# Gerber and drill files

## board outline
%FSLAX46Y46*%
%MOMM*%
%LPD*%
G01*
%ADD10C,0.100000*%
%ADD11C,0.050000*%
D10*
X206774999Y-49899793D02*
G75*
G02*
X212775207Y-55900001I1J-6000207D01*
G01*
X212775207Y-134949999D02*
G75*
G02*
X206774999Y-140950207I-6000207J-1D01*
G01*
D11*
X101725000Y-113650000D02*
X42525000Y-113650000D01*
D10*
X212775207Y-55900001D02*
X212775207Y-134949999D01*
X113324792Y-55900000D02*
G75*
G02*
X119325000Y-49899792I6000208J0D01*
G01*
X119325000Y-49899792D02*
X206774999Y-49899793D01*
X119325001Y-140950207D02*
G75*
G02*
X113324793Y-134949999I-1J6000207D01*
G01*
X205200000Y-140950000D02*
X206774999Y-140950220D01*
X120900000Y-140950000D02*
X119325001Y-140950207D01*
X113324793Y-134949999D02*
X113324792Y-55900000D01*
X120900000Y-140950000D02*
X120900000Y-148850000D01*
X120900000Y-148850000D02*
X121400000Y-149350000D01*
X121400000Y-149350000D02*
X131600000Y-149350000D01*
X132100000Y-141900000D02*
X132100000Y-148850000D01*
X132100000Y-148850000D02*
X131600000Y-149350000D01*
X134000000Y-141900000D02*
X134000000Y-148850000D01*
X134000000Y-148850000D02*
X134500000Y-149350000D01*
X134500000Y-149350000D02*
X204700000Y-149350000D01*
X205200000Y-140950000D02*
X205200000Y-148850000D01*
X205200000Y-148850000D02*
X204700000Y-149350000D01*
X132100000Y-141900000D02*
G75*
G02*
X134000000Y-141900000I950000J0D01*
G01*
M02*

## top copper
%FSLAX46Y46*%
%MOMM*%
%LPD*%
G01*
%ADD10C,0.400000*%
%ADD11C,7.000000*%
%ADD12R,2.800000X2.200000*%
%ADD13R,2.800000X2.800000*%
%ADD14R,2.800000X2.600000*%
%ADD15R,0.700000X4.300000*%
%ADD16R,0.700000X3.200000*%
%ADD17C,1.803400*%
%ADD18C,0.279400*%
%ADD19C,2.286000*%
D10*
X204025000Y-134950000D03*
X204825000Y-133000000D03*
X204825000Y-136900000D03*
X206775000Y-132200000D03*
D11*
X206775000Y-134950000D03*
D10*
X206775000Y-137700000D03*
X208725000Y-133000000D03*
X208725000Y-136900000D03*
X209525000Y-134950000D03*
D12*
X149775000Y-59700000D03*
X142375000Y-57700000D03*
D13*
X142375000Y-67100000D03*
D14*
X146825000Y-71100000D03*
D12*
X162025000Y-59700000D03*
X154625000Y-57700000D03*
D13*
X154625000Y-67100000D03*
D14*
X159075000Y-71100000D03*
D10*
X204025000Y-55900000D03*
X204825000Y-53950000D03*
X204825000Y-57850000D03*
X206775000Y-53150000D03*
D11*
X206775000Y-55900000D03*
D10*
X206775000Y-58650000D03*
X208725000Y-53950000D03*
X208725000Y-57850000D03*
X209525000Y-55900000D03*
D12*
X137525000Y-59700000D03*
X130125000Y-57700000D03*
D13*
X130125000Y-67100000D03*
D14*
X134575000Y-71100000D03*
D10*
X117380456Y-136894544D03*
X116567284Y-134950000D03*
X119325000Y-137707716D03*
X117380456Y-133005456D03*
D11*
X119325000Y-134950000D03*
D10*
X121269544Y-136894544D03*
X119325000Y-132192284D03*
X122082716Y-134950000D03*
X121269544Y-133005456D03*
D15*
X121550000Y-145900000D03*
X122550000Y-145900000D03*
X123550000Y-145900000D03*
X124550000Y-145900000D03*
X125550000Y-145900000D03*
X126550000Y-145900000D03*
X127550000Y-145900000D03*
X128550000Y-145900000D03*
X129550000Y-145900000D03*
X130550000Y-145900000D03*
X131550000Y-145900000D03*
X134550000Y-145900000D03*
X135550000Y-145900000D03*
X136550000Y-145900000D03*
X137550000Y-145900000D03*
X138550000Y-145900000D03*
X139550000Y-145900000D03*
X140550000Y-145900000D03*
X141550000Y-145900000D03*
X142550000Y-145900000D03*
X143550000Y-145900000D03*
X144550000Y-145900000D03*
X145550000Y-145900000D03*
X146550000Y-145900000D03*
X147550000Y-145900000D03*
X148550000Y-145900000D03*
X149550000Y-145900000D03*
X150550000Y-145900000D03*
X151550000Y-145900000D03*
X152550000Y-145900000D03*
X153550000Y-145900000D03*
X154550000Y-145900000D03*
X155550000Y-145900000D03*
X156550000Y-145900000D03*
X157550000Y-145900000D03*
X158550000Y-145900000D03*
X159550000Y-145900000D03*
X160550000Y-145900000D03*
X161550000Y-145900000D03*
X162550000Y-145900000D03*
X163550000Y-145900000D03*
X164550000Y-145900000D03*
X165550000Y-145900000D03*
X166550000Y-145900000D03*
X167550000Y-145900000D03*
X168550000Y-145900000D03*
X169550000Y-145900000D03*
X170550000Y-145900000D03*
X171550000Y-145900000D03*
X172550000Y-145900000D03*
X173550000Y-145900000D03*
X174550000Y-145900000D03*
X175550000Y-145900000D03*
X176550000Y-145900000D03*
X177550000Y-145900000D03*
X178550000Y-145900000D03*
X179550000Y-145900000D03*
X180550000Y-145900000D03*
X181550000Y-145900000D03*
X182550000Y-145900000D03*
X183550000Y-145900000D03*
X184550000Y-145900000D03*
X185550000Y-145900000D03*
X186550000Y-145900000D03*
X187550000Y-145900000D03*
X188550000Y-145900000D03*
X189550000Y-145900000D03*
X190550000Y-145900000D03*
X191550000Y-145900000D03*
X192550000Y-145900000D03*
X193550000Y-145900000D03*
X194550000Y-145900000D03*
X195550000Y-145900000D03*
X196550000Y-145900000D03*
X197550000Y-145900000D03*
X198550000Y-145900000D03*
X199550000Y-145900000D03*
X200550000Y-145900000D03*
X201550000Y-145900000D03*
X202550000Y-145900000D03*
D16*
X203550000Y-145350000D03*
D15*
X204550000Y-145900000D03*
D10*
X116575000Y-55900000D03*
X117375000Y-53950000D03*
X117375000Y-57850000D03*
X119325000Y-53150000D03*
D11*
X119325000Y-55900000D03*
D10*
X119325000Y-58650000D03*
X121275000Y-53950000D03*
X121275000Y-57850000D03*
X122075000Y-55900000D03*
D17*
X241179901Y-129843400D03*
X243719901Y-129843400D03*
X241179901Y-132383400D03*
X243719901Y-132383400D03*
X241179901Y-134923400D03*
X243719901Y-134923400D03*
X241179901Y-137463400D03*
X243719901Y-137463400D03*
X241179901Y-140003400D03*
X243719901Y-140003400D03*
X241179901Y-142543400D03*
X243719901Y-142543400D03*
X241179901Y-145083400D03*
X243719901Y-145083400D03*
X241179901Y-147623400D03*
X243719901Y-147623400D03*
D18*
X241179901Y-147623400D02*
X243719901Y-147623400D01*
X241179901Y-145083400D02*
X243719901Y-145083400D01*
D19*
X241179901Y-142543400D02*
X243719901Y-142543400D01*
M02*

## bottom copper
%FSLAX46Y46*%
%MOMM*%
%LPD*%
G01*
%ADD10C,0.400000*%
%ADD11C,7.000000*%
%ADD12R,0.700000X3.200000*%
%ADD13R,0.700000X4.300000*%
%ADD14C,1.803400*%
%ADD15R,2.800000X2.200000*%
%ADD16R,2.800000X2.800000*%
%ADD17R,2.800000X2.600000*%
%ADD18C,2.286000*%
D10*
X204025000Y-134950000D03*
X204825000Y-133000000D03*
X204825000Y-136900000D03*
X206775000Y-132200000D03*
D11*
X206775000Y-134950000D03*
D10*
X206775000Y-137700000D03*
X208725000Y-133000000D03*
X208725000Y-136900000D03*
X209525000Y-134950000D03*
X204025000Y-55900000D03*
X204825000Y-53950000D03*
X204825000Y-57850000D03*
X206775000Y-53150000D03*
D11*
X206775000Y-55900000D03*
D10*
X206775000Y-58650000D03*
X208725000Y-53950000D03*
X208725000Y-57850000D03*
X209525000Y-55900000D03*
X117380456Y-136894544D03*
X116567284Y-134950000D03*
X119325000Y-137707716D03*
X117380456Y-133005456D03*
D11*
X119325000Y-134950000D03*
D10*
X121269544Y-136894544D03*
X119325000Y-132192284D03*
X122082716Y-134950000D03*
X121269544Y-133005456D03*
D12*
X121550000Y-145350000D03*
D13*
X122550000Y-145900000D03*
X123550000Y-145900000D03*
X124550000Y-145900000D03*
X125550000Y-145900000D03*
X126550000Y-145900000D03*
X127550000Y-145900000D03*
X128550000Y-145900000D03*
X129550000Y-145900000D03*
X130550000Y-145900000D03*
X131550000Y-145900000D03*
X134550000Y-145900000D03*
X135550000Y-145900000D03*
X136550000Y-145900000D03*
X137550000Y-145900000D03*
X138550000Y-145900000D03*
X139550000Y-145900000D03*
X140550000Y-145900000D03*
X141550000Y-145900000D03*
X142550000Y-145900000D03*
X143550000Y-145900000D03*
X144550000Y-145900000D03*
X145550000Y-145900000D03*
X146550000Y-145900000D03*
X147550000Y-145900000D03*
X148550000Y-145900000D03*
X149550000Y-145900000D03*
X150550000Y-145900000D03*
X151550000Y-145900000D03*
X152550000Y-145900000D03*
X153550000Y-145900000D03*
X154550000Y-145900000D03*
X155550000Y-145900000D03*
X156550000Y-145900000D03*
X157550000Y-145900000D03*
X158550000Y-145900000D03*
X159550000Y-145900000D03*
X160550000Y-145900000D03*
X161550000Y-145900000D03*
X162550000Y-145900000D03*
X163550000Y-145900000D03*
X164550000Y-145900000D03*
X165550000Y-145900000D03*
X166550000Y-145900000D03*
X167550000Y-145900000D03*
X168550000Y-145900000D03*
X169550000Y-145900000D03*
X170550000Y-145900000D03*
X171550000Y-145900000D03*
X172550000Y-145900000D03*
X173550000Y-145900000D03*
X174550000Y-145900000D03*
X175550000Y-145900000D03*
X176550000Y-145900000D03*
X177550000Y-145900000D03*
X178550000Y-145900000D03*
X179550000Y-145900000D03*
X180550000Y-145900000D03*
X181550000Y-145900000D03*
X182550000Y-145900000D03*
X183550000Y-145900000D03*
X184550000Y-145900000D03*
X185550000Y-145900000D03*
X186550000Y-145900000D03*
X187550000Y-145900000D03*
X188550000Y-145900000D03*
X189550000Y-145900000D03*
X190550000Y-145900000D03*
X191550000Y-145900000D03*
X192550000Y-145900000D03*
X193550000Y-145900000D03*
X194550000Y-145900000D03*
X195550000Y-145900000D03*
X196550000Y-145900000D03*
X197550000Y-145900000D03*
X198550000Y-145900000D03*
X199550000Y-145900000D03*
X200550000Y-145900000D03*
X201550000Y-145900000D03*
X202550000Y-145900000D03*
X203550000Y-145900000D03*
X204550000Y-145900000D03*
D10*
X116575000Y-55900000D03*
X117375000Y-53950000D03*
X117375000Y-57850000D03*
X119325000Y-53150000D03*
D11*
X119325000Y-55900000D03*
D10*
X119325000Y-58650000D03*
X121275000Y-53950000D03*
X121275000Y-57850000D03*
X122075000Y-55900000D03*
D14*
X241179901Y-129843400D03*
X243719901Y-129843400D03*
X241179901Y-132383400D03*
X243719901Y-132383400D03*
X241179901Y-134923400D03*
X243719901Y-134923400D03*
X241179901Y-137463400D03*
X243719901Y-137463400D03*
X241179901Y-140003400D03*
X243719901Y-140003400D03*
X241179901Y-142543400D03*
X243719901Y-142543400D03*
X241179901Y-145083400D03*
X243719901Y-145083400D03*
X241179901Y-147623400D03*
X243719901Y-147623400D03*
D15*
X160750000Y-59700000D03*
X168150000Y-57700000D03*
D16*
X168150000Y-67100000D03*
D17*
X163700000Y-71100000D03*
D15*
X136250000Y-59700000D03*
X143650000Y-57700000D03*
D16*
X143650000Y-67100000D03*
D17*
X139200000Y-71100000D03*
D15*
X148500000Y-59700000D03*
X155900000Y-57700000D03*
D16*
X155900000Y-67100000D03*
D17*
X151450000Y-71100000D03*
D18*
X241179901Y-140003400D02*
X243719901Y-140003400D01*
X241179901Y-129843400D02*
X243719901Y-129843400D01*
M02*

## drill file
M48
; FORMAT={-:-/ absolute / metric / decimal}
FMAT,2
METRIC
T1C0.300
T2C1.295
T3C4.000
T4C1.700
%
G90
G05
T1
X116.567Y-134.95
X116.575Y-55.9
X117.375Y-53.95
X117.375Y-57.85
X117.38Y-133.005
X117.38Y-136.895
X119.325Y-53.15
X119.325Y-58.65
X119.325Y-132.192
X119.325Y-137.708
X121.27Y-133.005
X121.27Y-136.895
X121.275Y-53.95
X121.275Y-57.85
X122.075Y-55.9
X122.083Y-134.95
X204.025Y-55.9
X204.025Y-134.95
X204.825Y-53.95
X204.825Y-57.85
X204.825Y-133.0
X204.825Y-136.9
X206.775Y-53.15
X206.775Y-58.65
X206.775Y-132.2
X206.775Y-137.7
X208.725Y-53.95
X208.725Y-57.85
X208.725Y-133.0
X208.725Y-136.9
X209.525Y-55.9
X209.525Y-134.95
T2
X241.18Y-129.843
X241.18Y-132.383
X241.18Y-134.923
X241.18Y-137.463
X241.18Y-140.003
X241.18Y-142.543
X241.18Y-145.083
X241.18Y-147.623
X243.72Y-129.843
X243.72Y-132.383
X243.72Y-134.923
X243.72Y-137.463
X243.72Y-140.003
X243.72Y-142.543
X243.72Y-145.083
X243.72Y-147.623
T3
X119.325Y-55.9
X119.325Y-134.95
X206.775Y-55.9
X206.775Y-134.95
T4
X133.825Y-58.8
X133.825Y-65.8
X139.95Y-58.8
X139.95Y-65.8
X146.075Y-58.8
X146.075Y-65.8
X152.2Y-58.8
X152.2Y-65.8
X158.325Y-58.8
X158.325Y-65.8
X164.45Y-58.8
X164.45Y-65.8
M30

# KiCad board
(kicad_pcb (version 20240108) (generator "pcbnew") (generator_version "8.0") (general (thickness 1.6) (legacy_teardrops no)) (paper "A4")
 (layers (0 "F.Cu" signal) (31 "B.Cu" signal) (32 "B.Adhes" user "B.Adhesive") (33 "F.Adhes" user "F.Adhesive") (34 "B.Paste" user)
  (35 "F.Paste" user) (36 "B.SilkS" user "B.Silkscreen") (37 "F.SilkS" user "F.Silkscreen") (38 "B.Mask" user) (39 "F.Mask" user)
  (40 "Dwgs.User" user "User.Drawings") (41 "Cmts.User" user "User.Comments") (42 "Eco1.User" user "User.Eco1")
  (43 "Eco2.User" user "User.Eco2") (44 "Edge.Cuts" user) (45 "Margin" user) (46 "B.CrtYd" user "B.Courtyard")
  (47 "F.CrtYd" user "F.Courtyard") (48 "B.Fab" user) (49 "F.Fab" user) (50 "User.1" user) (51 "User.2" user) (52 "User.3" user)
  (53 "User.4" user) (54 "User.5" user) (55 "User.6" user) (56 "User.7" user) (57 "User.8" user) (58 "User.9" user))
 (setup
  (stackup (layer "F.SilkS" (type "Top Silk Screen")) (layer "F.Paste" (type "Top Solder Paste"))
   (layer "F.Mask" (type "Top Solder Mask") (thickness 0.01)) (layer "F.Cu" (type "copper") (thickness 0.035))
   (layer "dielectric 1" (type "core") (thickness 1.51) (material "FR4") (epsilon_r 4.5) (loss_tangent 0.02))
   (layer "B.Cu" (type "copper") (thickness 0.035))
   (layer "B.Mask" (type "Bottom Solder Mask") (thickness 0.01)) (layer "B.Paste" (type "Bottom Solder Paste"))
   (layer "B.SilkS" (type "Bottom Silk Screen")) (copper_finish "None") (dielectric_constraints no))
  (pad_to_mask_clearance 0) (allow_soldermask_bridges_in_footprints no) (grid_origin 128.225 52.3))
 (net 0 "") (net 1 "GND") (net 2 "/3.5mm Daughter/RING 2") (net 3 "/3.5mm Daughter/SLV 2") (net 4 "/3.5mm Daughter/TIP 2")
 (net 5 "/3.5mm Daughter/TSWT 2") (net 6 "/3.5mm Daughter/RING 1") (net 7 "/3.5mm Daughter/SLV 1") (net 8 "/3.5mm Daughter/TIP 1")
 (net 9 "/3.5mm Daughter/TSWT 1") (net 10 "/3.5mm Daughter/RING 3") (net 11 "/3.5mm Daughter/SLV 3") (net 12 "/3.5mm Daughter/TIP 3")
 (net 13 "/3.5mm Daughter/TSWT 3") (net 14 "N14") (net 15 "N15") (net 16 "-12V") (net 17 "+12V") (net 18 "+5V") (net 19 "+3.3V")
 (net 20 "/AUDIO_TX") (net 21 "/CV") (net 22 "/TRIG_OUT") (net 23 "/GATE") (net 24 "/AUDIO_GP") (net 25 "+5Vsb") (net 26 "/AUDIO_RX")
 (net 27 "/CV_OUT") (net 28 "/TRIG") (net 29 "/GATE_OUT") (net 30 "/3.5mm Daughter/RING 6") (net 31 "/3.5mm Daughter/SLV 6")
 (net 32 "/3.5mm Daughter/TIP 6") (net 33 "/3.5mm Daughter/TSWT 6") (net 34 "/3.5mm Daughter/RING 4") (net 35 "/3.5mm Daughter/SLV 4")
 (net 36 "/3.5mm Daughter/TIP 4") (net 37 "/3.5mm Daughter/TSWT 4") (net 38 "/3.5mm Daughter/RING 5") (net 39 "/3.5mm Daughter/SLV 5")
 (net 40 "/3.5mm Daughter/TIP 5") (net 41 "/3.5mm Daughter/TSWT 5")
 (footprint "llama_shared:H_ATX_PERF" (layer "F.Cu") (at 206.775 134.95)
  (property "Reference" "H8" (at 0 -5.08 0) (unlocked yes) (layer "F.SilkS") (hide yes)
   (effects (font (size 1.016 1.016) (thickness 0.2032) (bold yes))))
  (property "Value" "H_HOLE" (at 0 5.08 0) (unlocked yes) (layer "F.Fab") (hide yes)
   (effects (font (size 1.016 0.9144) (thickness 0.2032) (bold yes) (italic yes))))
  (pad "1" thru_hole circle (at -2.75 0) (size 0.4 0.4) (drill 0.3) (layers "*.Cu" "*.Mask") (remove_unused_layers no) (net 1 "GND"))
  (pad "1" thru_hole circle (at -1.95 -1.95) (size 0.4 0.4) (drill 0.3) (layers "*.Cu" "*.Mask") (remove_unused_layers no) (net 1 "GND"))
  (pad "1" thru_hole circle (at -1.95 1.95) (size 0.4 0.4) (drill 0.3) (layers "*.Cu" "*.Mask") (remove_unused_layers no) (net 1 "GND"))
  (pad "1" thru_hole circle (at 0 -2.75) (size 0.4 0.4) (drill 0.3) (layers "*.Cu" "*.Mask") (remove_unused_layers no) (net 1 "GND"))
  (pad "1" thru_hole circle (at 0 0) (size 7 7) (drill 4) (layers "*.Cu" "*.Mask") (remove_unused_layers no) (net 1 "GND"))
  (pad "1" thru_hole circle (at 0 2.75) (size 0.4 0.4) (drill 0.3) (layers "*.Cu" "*.Mask") (remove_unused_layers no) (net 1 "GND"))
  (pad "1" thru_hole circle (at 1.95 -1.95) (size 0.4 0.4) (drill 0.3) (layers "*.Cu" "*.Mask") (remove_unused_layers no) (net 1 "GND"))
  (pad "1" thru_hole circle (at 1.95 1.95) (size 0.4 0.4) (drill 0.3) (layers "*.Cu" "*.Mask") (remove_unused_layers no) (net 1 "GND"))
  (pad "1" thru_hole circle (at 2.75 0) (size 0.4 0.4) (drill 0.3) (layers "*.Cu" "*.Mask") (remove_unused_layers no) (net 1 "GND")))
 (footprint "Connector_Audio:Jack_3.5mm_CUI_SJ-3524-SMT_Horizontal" (layer "F.Cu") (at 146.075 61.3)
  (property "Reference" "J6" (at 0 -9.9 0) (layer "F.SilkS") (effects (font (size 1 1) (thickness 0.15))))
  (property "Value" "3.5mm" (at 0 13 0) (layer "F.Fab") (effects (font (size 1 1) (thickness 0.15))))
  (pad "" np_thru_hole circle (at 0 -2.5) (size 1.7 1.7) (drill 1.7) (layers "*.Cu" "*.Mask"))
  (pad "" np_thru_hole circle (at 0 4.5) (size 1.7 1.7) (drill 1.7) (layers "*.Cu" "*.Mask"))
  (pad "R" smd rect (at 3.7 -1.6) (size 2.8 2.2) (layers "F.Cu" "F.Paste" "F.Mask") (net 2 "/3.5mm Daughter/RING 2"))
  (pad "S" smd rect (at -3.7 -3.6) (size 2.8 2.2) (layers "F.Cu" "F.Paste" "F.Mask") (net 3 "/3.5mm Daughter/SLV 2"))
  (pad "T" smd rect (at -3.7 5.8) (size 2.8 2.8) (layers "F.Cu" "F.Paste" "F.Mask") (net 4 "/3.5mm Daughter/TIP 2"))
  (pad "TN" smd rect (at 0.75 9.8) (size 2.8 2.6) (layers "F.Cu" "F.Paste" "F.Mask") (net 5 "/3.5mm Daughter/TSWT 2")))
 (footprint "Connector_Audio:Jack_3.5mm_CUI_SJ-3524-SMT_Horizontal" (layer "F.Cu") (at 158.325 61.3)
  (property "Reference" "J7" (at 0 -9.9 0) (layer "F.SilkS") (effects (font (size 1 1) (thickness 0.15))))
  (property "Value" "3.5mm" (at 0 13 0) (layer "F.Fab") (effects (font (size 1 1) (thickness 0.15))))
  (pad "" np_thru_hole circle (at 0 -2.5) (size 1.7 1.7) (drill 1.7) (layers "*.Cu" "*.Mask"))
  (pad "" np_thru_hole circle (at 0 4.5) (size 1.7 1.7) (drill 1.7) (layers "*.Cu" "*.Mask"))
  (pad "R" smd rect (at 3.7 -1.6) (size 2.8 2.2) (layers "F.Cu" "F.Paste" "F.Mask") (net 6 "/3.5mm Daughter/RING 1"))
  (pad "S" smd rect (at -3.7 -3.6) (size 2.8 2.2) (layers "F.Cu" "F.Paste" "F.Mask") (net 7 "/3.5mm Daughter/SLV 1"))
  (pad "T" smd rect (at -3.7 5.8) (size 2.8 2.8) (layers "F.Cu" "F.Paste" "F.Mask") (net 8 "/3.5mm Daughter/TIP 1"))
  (pad "TN" smd rect (at 0.75 9.8) (size 2.8 2.6) (layers "F.Cu" "F.Paste" "F.Mask") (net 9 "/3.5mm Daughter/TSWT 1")))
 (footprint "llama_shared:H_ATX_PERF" (layer "F.Cu") (at 206.775 55.9)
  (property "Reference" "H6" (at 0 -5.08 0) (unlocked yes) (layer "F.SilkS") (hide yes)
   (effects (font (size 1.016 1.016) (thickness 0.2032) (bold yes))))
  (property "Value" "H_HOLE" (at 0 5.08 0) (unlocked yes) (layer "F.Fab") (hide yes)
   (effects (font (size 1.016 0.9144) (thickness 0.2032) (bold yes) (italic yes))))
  (pad "1" thru_hole circle (at -2.75 0) (size 0.4 0.4) (drill 0.3) (layers "*.Cu" "*.Mask") (remove_unused_layers no) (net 1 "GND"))
  (pad "1" thru_hole circle (at -1.95 -1.95) (size 0.4 0.4) (drill 0.3) (layers "*.Cu" "*.Mask") (remove_unused_layers no) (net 1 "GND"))
  (pad "1" thru_hole circle (at -1.95 1.95) (size 0.4 0.4) (drill 0.3) (layers "*.Cu" "*.Mask") (remove_unused_layers no) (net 1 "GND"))
  (pad "1" thru_hole circle (at 0 -2.75) (size 0.4 0.4) (drill 0.3) (layers "*.Cu" "*.Mask") (remove_unused_layers no) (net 1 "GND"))
  (pad "1" thru_hole circle (at 0 0) (size 7 7) (drill 4) (layers "*.Cu" "*.Mask") (remove_unused_layers no) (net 1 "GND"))
  (pad "1" thru_hole circle (at 0 2.75) (size 0.4 0.4) (drill 0.3) (layers "*.Cu" "*.Mask") (remove_unused_layers no) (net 1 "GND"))
  (pad "1" thru_hole circle (at 1.95 -1.95) (size 0.4 0.4) (drill 0.3) (layers "*.Cu" "*.Mask") (remove_unused_layers no) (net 1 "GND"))
  (pad "1" thru_hole circle (at 1.95 1.95) (size 0.4 0.4) (drill 0.3) (layers "*.Cu" "*.Mask") (remove_unused_layers no) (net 1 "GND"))
  (pad "1" thru_hole circle (at 2.75 0) (size 0.4 0.4) (drill 0.3) (layers "*.Cu" "*.Mask") (remove_unused_layers no) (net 1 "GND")))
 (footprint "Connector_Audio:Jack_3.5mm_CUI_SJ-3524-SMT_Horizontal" (layer "F.Cu") (at 133.825 61.3)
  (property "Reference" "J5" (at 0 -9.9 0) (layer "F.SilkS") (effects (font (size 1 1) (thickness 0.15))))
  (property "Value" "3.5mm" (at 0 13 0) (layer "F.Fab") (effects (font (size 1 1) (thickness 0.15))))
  (pad "" np_thru_hole circle (at 0 -2.5) (size 1.7 1.7) (drill 1.7) (layers "*.Cu" "*.Mask"))
  (pad "" np_thru_hole circle (at 0 4.5) (size 1.7 1.7) (drill 1.7) (layers "*.Cu" "*.Mask"))
  (pad "R" smd rect (at 3.7 -1.6) (size 2.8 2.2) (layers "F.Cu" "F.Paste" "F.Mask") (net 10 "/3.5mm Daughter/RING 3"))
  (pad "S" smd rect (at -3.7 -3.6) (size 2.8 2.2) (layers "F.Cu" "F.Paste" "F.Mask") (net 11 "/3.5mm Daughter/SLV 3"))
  (pad "T" smd rect (at -3.7 5.8) (size 2.8 2.8) (layers "F.Cu" "F.Paste" "F.Mask") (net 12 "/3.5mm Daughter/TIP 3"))
  (pad "TN" smd rect (at 0.75 9.8) (size 2.8 2.6) (layers "F.Cu" "F.Paste" "F.Mask") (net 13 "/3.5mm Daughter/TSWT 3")))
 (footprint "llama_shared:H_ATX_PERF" (layer "F.Cu") (at 119.325 134.95 45)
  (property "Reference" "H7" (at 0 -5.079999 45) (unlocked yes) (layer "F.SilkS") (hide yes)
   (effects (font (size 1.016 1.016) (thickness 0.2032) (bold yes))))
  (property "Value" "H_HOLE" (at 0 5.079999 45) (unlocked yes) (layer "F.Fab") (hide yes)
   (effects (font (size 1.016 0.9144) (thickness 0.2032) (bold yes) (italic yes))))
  (pad "1" thru_hole circle (at -2.75 0 45) (size 0.4 0.4) (drill 0.3) (layers "*.Cu" "*.Mask") (remove_unused_layers no) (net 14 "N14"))
  (pad "1" thru_hole circle (at -1.95 -1.95 45) (size 0.4 0.4) (drill 0.3) (layers "*.Cu" "*.Mask") (remove_unused_layers no) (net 14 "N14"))
  (pad "1" thru_hole circle (at -1.95 1.95 45) (size 0.4 0.4) (drill 0.3) (layers "*.Cu" "*.Mask") (remove_unused_layers no) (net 14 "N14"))
  (pad "1" thru_hole circle (at 0 -2.75 45) (size 0.4 0.4) (drill 0.3) (layers "*.Cu" "*.Mask") (remove_unused_layers no) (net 14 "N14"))
  (pad "1" thru_hole circle (at 0 0 45) (size 7 7) (drill 4) (layers "*.Cu" "*.Mask") (remove_unused_layers no) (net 14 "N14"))
  (pad "1" thru_hole circle (at 0 2.75 45) (size 0.4 0.4) (drill 0.3) (layers "*.Cu" "*.Mask") (remove_unused_layers no) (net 14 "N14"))
  (pad "1" thru_hole circle (at 1.95 -1.95 45) (size 0.4 0.4) (drill 0.3) (layers "*.Cu" "*.Mask") (remove_unused_layers no) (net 14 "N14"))
  (pad "1" thru_hole circle (at 1.95 1.95 45) (size 0.4 0.4) (drill 0.3) (layers "*.Cu" "*.Mask") (remove_unused_layers no) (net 14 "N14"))
  (pad "1" thru_hole circle (at 2.75 0 45) (size 0.4 0.4) (drill 0.3) (layers "*.Cu" "*.Mask") (remove_unused_layers no) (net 14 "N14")))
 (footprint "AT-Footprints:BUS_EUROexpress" (layer "F.Cu") (at 121.55 145.9)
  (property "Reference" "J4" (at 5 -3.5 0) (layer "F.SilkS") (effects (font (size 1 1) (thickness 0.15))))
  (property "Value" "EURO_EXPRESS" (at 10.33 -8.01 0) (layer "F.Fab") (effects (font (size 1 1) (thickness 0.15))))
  (fp_line (start -0.65 -4.95) (end -0.65 2.95) (stroke (width 0.1) (type solid)) (layer "Edge.Cuts"))
  (fp_line (start -0.65 2.95) (end -0.15 3.45) (stroke (width 0.1) (type solid)) (layer "Edge.Cuts"))
  (fp_line (start -0.15 3.45) (end 10.05 3.45) (stroke (width 0.1) (type solid)) (layer "Edge.Cuts"))
  (fp_line (start 10.55 -4) (end 10.55 2.95) (stroke (width 0.1) (type solid)) (layer "Edge.Cuts"))
  (fp_line (start 10.55 2.95) (end 10.05 3.45) (stroke (width 0.1) (type solid)) (layer "Edge.Cuts"))
  (fp_line (start 12.45 -4) (end 12.45 2.95) (stroke (width 0.1) (type solid)) (layer "Edge.Cuts"))
  (fp_line (start 12.45 2.95) (end 12.95 3.45) (stroke (width 0.1) (type solid)) (layer "Edge.Cuts"))
  (fp_line (start 12.95 3.45) (end 83.15 3.45) (stroke (width 0.1) (type solid)) (layer "Edge.Cuts"))
  (fp_line (start 83.65 -4.95) (end 83.65 2.95) (stroke (width 0.1) (type solid)) (layer "Edge.Cuts"))
  (fp_line (start 83.65 2.95) (end 83.15 3.45) (stroke (width 0.1) (type solid)) (layer "Edge.Cuts"))
  (fp_arc (start 10.55 -4) (mid 11.5 -4.95) (end 12.45 -4) (stroke (width 0.1) (type solid)) (layer "Edge.Cuts"))
  (pad "A1" connect rect (at 0 -0.55) (size 0.7 3.2) (layers "B.Cu" "B.Mask") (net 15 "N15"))
  (pad "A2" connect rect (at 1 0) (size 0.7 4.3) (layers "B.Cu" "B.Mask") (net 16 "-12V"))
  (pad "A3" connect rect (at 2 0) (size 0.7 4.3) (layers "B.Cu" "B.Mask") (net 16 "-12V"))
  (pad "A4" connect rect (at 3 0) (size 0.7 4.3) (layers "B.Cu" "B.Mask") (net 1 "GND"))
  (pad "A5" connect rect (at 4 0) (size 0.7 4.3) (layers "B.Cu" "B.Mask") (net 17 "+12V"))
  (pad "A6" connect rect (at 5 0) (size 0.7 4.3) (layers "B.Cu" "B.Mask") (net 17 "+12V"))
  (pad "A7" connect rect (at 6 0) (size 0.7 4.3) (layers "B.Cu" "B.Mask") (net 17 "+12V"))
  (pad "A8" connect rect (at 7 0) (size 0.7 4.3) (layers "B.Cu" "B.Mask") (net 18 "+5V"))
  (pad "A9" connect rect (at 8 0) (size 0.7 4.3) (layers "B.Cu" "B.Mask") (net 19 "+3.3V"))
  (pad "A10" connect rect (at 9 0) (size 0.7 4.3) (layers "B.Cu" "B.Mask") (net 19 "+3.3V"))
  (pad "A11" connect rect (at 10 0) (size 0.7 4.3) (layers "B.Cu" "B.Mask") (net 1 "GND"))
  (pad "A12" connect rect (at 13 0) (size 0.7 4.3) (layers "B.Cu" "B.Mask") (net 1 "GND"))
  (pad "A13" connect rect (at 14 0) (size 0.7 4.3) (layers "B.Cu" "B.Mask") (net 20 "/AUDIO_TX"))
  (pad "A14" connect rect (at 15 0) (size 0.7 4.3) (layers "B.Cu" "B.Mask") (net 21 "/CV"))
  (pad "A15" connect rect (at 16 0) (size 0.7 4.3) (layers "B.Cu" "B.Mask") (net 1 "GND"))
  (pad "A16" connect rect (at 17 0) (size 0.7 4.3) (layers "B.Cu" "B.Mask") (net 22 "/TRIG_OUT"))
  (pad "A17" connect rect (at 18 0) (size 0.7 4.3) (layers "B.Cu" "B.Mask") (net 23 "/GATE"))
  (pad "A18" connect rect (at 19 0) (size 0.7 4.3) (layers "B.Cu" "B.Mask") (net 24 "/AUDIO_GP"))
  (pad "A19" connect rect (at 20 0) (size 0.7 4.3) (layers "B.Cu" "B.Mask"))
  (pad "A20" connect rect (at 21 0) (size 0.7 4.3) (layers "B.Cu" "B.Mask"))
  (pad "A21" connect rect (at 22 0) (size 0.7 4.3) (layers "B.Cu" "B.Mask"))
  (pad "A22" connect rect (at 23 0) (size 0.7 4.3) (layers "B.Cu" "B.Mask"))
  (pad "A23" connect rect (at 24 0) (size 0.7 4.3) (layers "B.Cu" "B.Mask"))
  (pad "A24" connect rect (at 25 0) (size 0.7 4.3) (layers "B.Cu" "B.Mask"))
  (pad "A25" connect rect (at 26 0) (size 0.7 4.3) (layers "B.Cu" "B.Mask"))
  (pad "A26" connect rect (at 27 0) (size 0.7 4.3) (layers "B.Cu" "B.Mask"))
  (pad "A27" connect rect (at 28 0) (size 0.7 4.3) (layers "B.Cu" "B.Mask"))
  (pad "A28" connect rect (at 29 0) (size 0.7 4.3) (layers "B.Cu" "B.Mask"))
  (pad "A29" connect rect (at 30 0) (size 0.7 4.3) (layers "B.Cu" "B.Mask"))
  (pad "A30" connect rect (at 31 0) (size 0.7 4.3) (layers "B.Cu" "B.Mask"))
  (pad "A31" connect rect (at 32 0) (size 0.7 4.3) (layers "B.Cu" "B.Mask"))
  (pad "A32" connect rect (at 33 0) (size 0.7 4.3) (layers "B.Cu" "B.Mask"))
  (pad "A33" connect rect (at 34 0) (size 0.7 4.3) (layers "B.Cu" "B.Mask"))
  (pad "A34" connect rect (at 35 0) (size 0.7 4.3) (layers "B.Cu" "B.Mask"))
  (pad "A35" connect rect (at 36 0) (size 0.7 4.3) (layers "B.Cu" "B.Mask"))
  (pad "A36" connect rect (at 37 0) (size 0.7 4.3) (layers "B.Cu" "B.Mask"))
  (pad "A37" connect rect (at 38 0) (size 0.7 4.3) (layers "B.Cu" "B.Mask"))
  (pad "A38" connect rect (at 39 0) (size 0.7 4.3) (layers "B.Cu" "B.Mask"))
  (pad "A39" connect rect (at 40 0) (size 0.7 4.3) (layers "B.Cu" "B.Mask"))
  (pad "A40" connect rect (at 41 0) (size 0.7 4.3) (layers "B.Cu" "B.Mask"))
  (pad "A41" connect rect (at 42 0) (size 0.7 4.3) (layers "B.Cu" "B.Mask"))
  (pad "A42" connect rect (at 43 0) (size 0.7 4.3) (layers "B.Cu" "B.Mask"))
  (pad "A43" connect rect (at 44 0) (size 0.7 4.3) (layers "B.Cu" "B.Mask"))
  (pad "A44" connect rect (at 45 0) (size 0.7 4.3) (layers "B.Cu" "B.Mask"))
  (pad "A45" connect rect (at 46 0) (size 0.7 4.3) (layers "B.Cu" "B.Mask"))
  (pad "A46" connect rect (at 47 0) (size 0.7 4.3) (layers "B.Cu" "B.Mask"))
  (pad "A47" connect rect (at 48 0) (size 0.7 4.3) (layers "B.Cu" "B.Mask"))
  (pad "A48" connect rect (at 49 0) (size 0.7 4.3) (layers "B.Cu" "B.Mask"))
  (pad "A49" connect rect (at 50 0) (size 0.7 4.3) (layers "B.Cu" "B.Mask"))
  (pad "A50" connect rect (at 51 0) (size 0.7 4.3) (layers "B.Cu" "B.Mask"))
  (pad "A51" connect rect (at 52 0) (size 0.7 4.3) (layers "B.Cu" "B.Mask"))
  (pad "A52" connect rect (at 53 0) (size 0.7 4.3) (layers "B.Cu" "B.Mask"))
  (pad "A53" connect rect (at 54 0) (size 0.7 4.3) (layers "B.Cu" "B.Mask"))
  (pad "A54" connect rect (at 55 0) (size 0.7 4.3) (layers "B.Cu" "B.Mask"))
  (pad "A55" connect rect (at 56 0) (size 0.7 4.3) (layers "B.Cu" "B.Mask"))
  (pad "A56" connect rect (at 57 0) (size 0.7 4.3) (layers "B.Cu" "B.Mask"))
  (pad "A57" connect rect (at 58 0) (size 0.7 4.3) (layers "B.Cu" "B.Mask"))
  (pad "A58" connect rect (at 59 0) (size 0.7 4.3) (layers "B.Cu" "B.Mask"))
  (pad "A59" connect rect (at 60 0) (size 0.7 4.3) (layers "B.Cu" "B.Mask"))
  (pad "A60" connect rect (at 61 0) (size 0.7 4.3) (layers "B.Cu" "B.Mask"))
  (pad "A61" connect rect (at 62 0) (size 0.7 4.3) (layers "B.Cu" "B.Mask"))
  (pad "A62" connect rect (at 63 0) (size 0.7 4.3) (layers "B.Cu" "B.Mask"))
  (pad "A63" connect rect (at 64 0) (size 0.7 4.3) (layers "B.Cu" "B.Mask"))
  (pad "A64" connect rect (at 65 0) (size 0.7 4.3) (layers "B.Cu" "B.Mask"))
  (pad "A65" connect rect (at 66 0) (size 0.7 4.3) (layers "B.Cu" "B.Mask"))
  (pad "A66" connect rect (at 67 0) (size 0.7 4.3) (layers "B.Cu" "B.Mask"))
  (pad "A67" connect rect (at 68 0) (size 0.7 4.3) (layers "B.Cu" "B.Mask"))
  (pad "A68" connect rect (at 69 0) (size 0.7 4.3) (layers "B.Cu" "B.Mask"))
  (pad "A69" connect rect (at 70 0) (size 0.7 4.3) (layers "B.Cu" "B.Mask"))
  (pad "A70" connect rect (at 71 0) (size 0.7 4.3) (layers "B.Cu" "B.Mask"))
  (pad "A71" connect rect (at 72 0) (size 0.7 4.3) (layers "B.Cu" "B.Mask"))
  (pad "A72" connect rect (at 73 0) (size 0.7 4.3) (layers "B.Cu" "B.Mask"))
  (pad "A73" connect rect (at 74 0) (size 0.7 4.3) (layers "B.Cu" "B.Mask"))
  (pad "A74" connect rect (at 75 0) (size 0.7 4.3) (layers "B.Cu" "B.Mask"))
  (pad "A75" connect rect (at 76 0) (size 0.7 4.3) (layers "B.Cu" "B.Mask"))
  (pad "A76" connect rect (at 77 0) (size 0.7 4.3) (layers "B.Cu" "B.Mask"))
  (pad "A77" connect rect (at 78 0) (size 0.7 4.3) (layers "B.Cu" "B.Mask"))
  (pad "A78" connect rect (at 79 0) (size 0.7 4.3) (layers "B.Cu" "B.Mask"))
  (pad "A79" connect rect (at 80 0) (size 0.7 4.3) (layers "B.Cu" "B.Mask"))
  (pad "A80" connect rect (at 81 0) (size 0.7 4.3) (layers "B.Cu" "B.Mask"))
  (pad "A81" connect rect (at 82 0) (size 0.7 4.3) (layers "B.Cu" "B.Mask"))
  (pad "A82" connect rect (at 83 0) (size 0.7 4.3) (layers "B.Cu" "B.Mask"))
  (pad "B1" connect rect (at 0 0) (size 0.7 4.3) (layers "F.Cu" "F.Mask") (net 16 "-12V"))
  (pad "B2" connect rect (at 1 0) (size 0.7 4.3) (layers "F.Cu" "F.Mask") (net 16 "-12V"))
  (pad "B3" connect rect (at 2 0) (size 0.7 4.3) (layers "F.Cu" "F.Mask") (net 16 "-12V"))
  (pad "B4" connect rect (at 3 0) (size 0.7 4.3) (layers "F.Cu" "F.Mask") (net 1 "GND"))
  (pad "B5" connect rect (at 4 0) (size 0.7 4.3) (layers "F.Cu" "F.Mask") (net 17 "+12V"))
  (pad "B6" connect rect (at 5 0) (size 0.7 4.3) (layers "F.Cu" "F.Mask") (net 17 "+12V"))
  (pad "B7" connect rect (at 6 0) (size 0.7 4.3) (layers "F.Cu" "F.Mask") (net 1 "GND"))
  (pad "B8" connect rect (at 7 0) (size 0.7 4.3) (layers "F.Cu" "F.Mask") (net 19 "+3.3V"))
  (pad "B9" connect rect (at 8 0) (size 0.7 4.3) (layers "F.Cu" "F.Mask") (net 18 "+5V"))
  (pad "B10" connect rect (at 9 0) (size 0.7 4.3) (layers "F.Cu" "F.Mask") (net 18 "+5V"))
  (pad "B11" connect rect (at 10 0) (size 0.7 4.3) (layers "F.Cu" "F.Mask") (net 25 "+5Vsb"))
  (pad "B12" connect rect (at 13 0) (size 0.7 4.3) (layers "F.Cu" "F.Mask") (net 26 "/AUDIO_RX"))
  (pad "B13" connect rect (at 14 0) (size 0.7 4.3) (layers "F.Cu" "F.Mask") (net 1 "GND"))
  (pad "B14" connect rect (at 15 0) (size 0.7 4.3) (layers "F.Cu" "F.Mask") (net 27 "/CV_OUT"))
  (pad "B15" connect rect (at 16 0) (size 0.7 4.3) (layers "F.Cu" "F.Mask") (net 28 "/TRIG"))
  (pad "B16" connect rect (at 17 0) (size 0.7 4.3) (layers "F.Cu" "F.Mask") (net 1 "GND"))
  (pad "B17" connect rect (at 18 0) (size 0.7 4.3) (layers "F.Cu" "F.Mask") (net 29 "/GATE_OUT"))
  (pad "B18" connect rect (at 19 0) (size 0.7 4.3) (layers "F.Cu" "F.Mask") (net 1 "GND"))
  (pad "B19" connect rect (at 20 0) (size 0.7 4.3) (layers "F.Cu" "F.Mask"))
  (pad "B20" connect rect (at 21 0) (size 0.7 4.3) (layers "F.Cu" "F.Mask"))
  (pad "B21" connect rect (at 22 0) (size 0.7 4.3) (layers "F.Cu" "F.Mask"))
  (pad "B22" connect rect (at 23 0) (size 0.7 4.3) (layers "F.Cu" "F.Mask"))
  (pad "B23" connect rect (at 24 0) (size 0.7 4.3) (layers "F.Cu" "F.Mask"))
  (pad "B24" connect rect (at 25 0) (size 0.7 4.3) (layers "F.Cu" "F.Mask"))
  (pad "B25" connect rect (at 26 0) (size 0.7 4.3) (layers "F.Cu" "F.Mask"))
  (pad "B26" connect rect (at 27 0) (size 0.7 4.3) (layers "F.Cu" "F.Mask"))
  (pad "B27" connect rect (at 28 0) (size 0.7 4.3) (layers "F.Cu" "F.Mask"))
  (pad "B28" connect rect (at 29 0) (size 0.7 4.3) (layers "F.Cu" "F.Mask"))
  (pad "B29" connect rect (at 30 0) (size 0.7 4.3) (layers "F.Cu" "F.Mask"))
  (pad "B30" connect rect (at 31 0) (size 0.7 4.3) (layers "F.Cu" "F.Mask"))
  (pad "B31" connect rect (at 32 0) (size 0.7 4.3) (layers "F.Cu" "F.Mask"))
  (pad "B32" connect rect (at 33 0) (size 0.7 4.3) (layers "F.Cu" "F.Mask"))
  (pad "B33" connect rect (at 34 0) (size 0.7 4.3) (layers "F.Cu" "F.Mask"))
  (pad "B34" connect rect (at 35 0) (size 0.7 4.3) (layers "F.Cu" "F.Mask"))
  (pad "B35" connect rect (at 36 0) (size 0.7 4.3) (layers "F.Cu" "F.Mask"))
  (pad "B36" connect rect (at 37 0) (size 0.7 4.3) (layers "F.Cu" "F.Mask"))
  (pad "B37" connect rect (at 38 0) (size 0.7 4.3) (layers "F.Cu" "F.Mask"))
  (pad "B38" connect rect (at 39 0) (size 0.7 4.3) (layers "F.Cu" "F.Mask"))
  (pad "B39" connect rect (at 40 0) (size 0.7 4.3) (layers "F.Cu" "F.Mask"))
  (pad "B40" connect rect (at 41 0) (size 0.7 4.3) (layers "F.Cu" "F.Mask"))
  (pad "B41" connect rect (at 42 0) (size 0.7 4.3) (layers "F.Cu" "F.Mask"))
  (pad "B42" connect rect (at 43 0) (size 0.7 4.3) (layers "F.Cu" "F.Mask"))
  (pad "B43" connect rect (at 44 0) (size 0.7 4.3) (layers "F.Cu" "F.Mask"))
  (pad "B44" connect rect (at 45 0) (size 0.7 4.3) (layers "F.Cu" "F.Mask"))
  (pad "B45" connect rect (at 46 0) (size 0.7 4.3) (layers "F.Cu" "F.Mask"))
  (pad "B46" connect rect (at 47 0) (size 0.7 4.3) (layers "F.Cu" "F.Mask"))
  (pad "B47" connect rect (at 48 0) (size 0.7 4.3) (layers "F.Cu" "F.Mask"))
  (pad "B48" connect rect (at 49 0) (size 0.7 4.3) (layers "F.Cu" "F.Mask"))
  (pad "B49" connect rect (at 50 0) (size 0.7 4.3) (layers "F.Cu" "F.Mask"))
  (pad "B50" connect rect (at 51 0) (size 0.7 4.3) (layers "F.Cu" "F.Mask"))
  (pad "B51" connect rect (at 52 0) (size 0.7 4.3) (layers "F.Cu" "F.Mask"))
  (pad "B52" connect rect (at 53 0) (size 0.7 4.3) (layers "F.Cu" "F.Mask"))
  (pad "B53" connect rect (at 54 0) (size 0.7 4.3) (layers "F.Cu" "F.Mask"))
  (pad "B54" connect rect (at 55 0) (size 0.7 4.3) (layers "F.Cu" "F.Mask"))
  (pad "B55" connect rect (at 56 0) (size 0.7 4.3) (layers "F.Cu" "F.Mask"))
  (pad "B56" connect rect (at 57 0) (size 0.7 4.3) (layers "F.Cu" "F.Mask"))
  (pad "B57" connect rect (at 58 0) (size 0.7 4.3) (layers "F.Cu" "F.Mask"))
  (pad "B58" connect rect (at 59 0) (size 0.7 4.3) (layers "F.Cu" "F.Mask"))
  (pad "B59" connect rect (at 60 0) (size 0.7 4.3) (layers "F.Cu" "F.Mask"))
  (pad "B60" connect rect (at 61 0) (size 0.7 4.3) (layers "F.Cu" "F.Mask"))
  (pad "B61" connect rect (at 62 0) (size 0.7 4.3) (layers "F.Cu" "F.Mask"))
  (pad "B62" connect rect (at 63 0) (size 0.7 4.3) (layers "F.Cu" "F.Mask"))
  (pad "B63" connect rect (at 64 0) (size 0.7 4.3) (layers "F.Cu" "F.Mask"))
  (pad "B64" connect rect (at 65 0) (size 0.7 4.3) (layers "F.Cu" "F.Mask"))
  (pad "B65" connect rect (at 66 0) (size 0.7 4.3) (layers "F.Cu" "F.Mask"))
  (pad "B66" connect rect (at 67 0) (size 0.7 4.3) (layers "F.Cu" "F.Mask"))
  (pad "B67" connect rect (at 68 0) (size 0.7 4.3) (layers "F.Cu" "F.Mask"))
  (pad "B68" connect rect (at 69 0) (size 0.7 4.3) (layers "F.Cu" "F.Mask"))
  (pad "B69" connect rect (at 70 0) (size 0.7 4.3) (layers "F.Cu" "F.Mask"))
  (pad "B70" connect rect (at 71 0) (size 0.7 4.3) (layers "F.Cu" "F.Mask"))
  (pad "B71" connect rect (at 72 0) (size 0.7 4.3) (layers "F.Cu" "F.Mask"))
  (pad "B72" connect rect (at 73 0) (size 0.7 4.3) (layers "F.Cu" "F.Mask"))
  (pad "B73" connect rect (at 74 0) (size 0.7 4.3) (layers "F.Cu" "F.Mask"))
  (pad "B74" connect rect (at 75 0) (size 0.7 4.3) (layers "F.Cu" "F.Mask"))
  (pad "B75" connect rect (at 76 0) (size 0.7 4.3) (layers "F.Cu" "F.Mask"))
  (pad "B76" connect rect (at 77 0) (size 0.7 4.3) (layers "F.Cu" "F.Mask"))
  (pad "B77" connect rect (at 78 0) (size 0.7 4.3) (layers "F.Cu" "F.Mask"))
  (pad "B78" connect rect (at 79 0) (size 0.7 4.3) (layers "F.Cu" "F.Mask"))
  (pad "B79" connect rect (at 80 0) (size 0.7 4.3) (layers "F.Cu" "F.Mask"))
  (pad "B80" connect rect (at 81 0) (size 0.7 4.3) (layers "F.Cu" "F.Mask"))
  (pad "B81" connect rect (at 82 -0.55) (size 0.7 3.2) (layers "F.Cu" "F.Mask"))
  (pad "B82" connect rect (at 83 0) (size 0.7 4.3) (layers "F.Cu" "F.Mask")))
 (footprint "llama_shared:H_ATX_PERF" (layer "F.Cu") (at 119.325 55.9)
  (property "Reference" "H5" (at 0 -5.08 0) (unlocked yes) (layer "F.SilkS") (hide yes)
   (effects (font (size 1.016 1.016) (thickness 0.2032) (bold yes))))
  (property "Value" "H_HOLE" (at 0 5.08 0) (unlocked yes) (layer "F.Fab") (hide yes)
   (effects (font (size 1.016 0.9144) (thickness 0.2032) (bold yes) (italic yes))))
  (pad "1" thru_hole circle (at -2.75 0) (size 0.4 0.4) (drill 0.3) (layers "*.Cu" "*.Mask") (remove_unused_layers no) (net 1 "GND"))
  (pad "1" thru_hole circle (at -1.95 -1.95) (size 0.4 0.4) (drill 0.3) (layers "*.Cu" "*.Mask") (remove_unused_layers no) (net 1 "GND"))
  (pad "1" thru_hole circle (at -1.95 1.95) (size 0.4 0.4) (drill 0.3) (layers "*.Cu" "*.Mask") (remove_unused_layers no) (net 1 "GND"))
  (pad "1" thru_hole circle (at 0 -2.75) (size 0.4 0.4) (drill 0.3) (layers "*.Cu" "*.Mask") (remove_unused_layers no) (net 1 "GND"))
  (pad "1" thru_hole circle (at 0 0) (size 7 7) (drill 4) (layers "*.Cu" "*.Mask") (remove_unused_layers no) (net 1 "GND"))
  (pad "1" thru_hole circle (at 0 2.75) (size 0.4 0.4) (drill 0.3) (layers "*.Cu" "*.Mask") (remove_unused_layers no) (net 1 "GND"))
  (pad "1" thru_hole circle (at 1.95 -1.95) (size 0.4 0.4) (drill 0.3) (layers "*.Cu" "*.Mask") (remove_unused_layers no) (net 1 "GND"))
  (pad "1" thru_hole circle (at 1.95 1.95) (size 0.4 0.4) (drill 0.3) (layers "*.Cu" "*.Mask") (remove_unused_layers no) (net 1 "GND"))
  (pad "1" thru_hole circle (at 2.75 0) (size 0.4 0.4) (drill 0.3) (layers "*.Cu" "*.Mask") (remove_unused_layers no) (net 1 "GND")))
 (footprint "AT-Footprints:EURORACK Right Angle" (layer "F.Cu") (at 241.179901 129.8434 -90)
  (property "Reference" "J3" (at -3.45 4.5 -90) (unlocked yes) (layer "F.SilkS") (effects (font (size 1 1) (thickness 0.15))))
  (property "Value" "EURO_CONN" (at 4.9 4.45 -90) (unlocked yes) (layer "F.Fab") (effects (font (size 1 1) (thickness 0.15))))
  (pad "1" thru_hole circle (at 0 0 270) (size 1.8034 1.8034) (drill 1.2954) (layers "*.Cu" "*.Mask") (remove_unused_layers no)
   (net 16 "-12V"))
  (pad "2" thru_hole circle (at 0 -2.54 270) (size 1.8034 1.8034) (drill 1.2954) (layers "*.Cu" "*.Mask") (remove_unused_layers no)
   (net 16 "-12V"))
  (pad "3" thru_hole circle (at 2.54 0 270) (size 1.8034 1.8034) (drill 1.2954) (layers "*.Cu" "*.Mask") (remove_unused_layers no)
   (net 1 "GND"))
  (pad "4" thru_hole circle (at 2.54 -2.54 270) (size 1.8034 1.8034) (drill 1.2954) (layers "*.Cu" "*.Mask") (remove_unused_layers no)
   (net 1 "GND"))
  (pad "5" thru_hole circle (at 5.08 0 270) (size 1.8034 1.8034) (drill 1.2954) (layers "*.Cu" "*.Mask") (remove_unused_layers no)
   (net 1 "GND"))
  (pad "6" thru_hole circle (at 5.08 -2.54 270) (size 1.8034 1.8034) (drill 1.2954) (layers "*.Cu" "*.Mask") (remove_unused_layers no)
   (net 1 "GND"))
  (pad "7" thru_hole circle (at 7.62 0 270) (size 1.8034 1.8034) (drill 1.2954) (layers "*.Cu" "*.Mask") (remove_unused_layers no)
   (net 1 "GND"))
  (pad "8" thru_hole circle (at 7.62 -2.54 270) (size 1.8034 1.8034) (drill 1.2954) (layers "*.Cu" "*.Mask") (remove_unused_layers no)
   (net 1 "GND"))
  (pad "9" thru_hole circle (at 10.16 0 270) (size 1.8034 1.8034) (drill 1.2954) (layers "*.Cu" "*.Mask") (remove_unused_layers no)
   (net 17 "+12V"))
  (pad "10" thru_hole circle (at 10.16 -2.54 270) (size 1.8034 1.8034) (drill 1.2954) (layers "*.Cu" "*.Mask") (remove_unused_layers no)
   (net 17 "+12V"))
  (pad "11" thru_hole circle (at 12.7 0 270) (size 1.8034 1.8034) (drill 1.2954) (layers "*.Cu" "*.Mask") (remove_unused_layers no)
   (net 18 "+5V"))
  (pad "12" thru_hole circle (at 12.7 -2.54 270) (size 1.8034 1.8034) (drill 1.2954) (layers "*.Cu" "*.Mask") (remove_unused_layers no)
   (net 18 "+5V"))
  (pad "13" thru_hole circle (at 15.24 0 270) (size 1.8034 1.8034) (drill 1.2954) (layers "*.Cu" "*.Mask") (remove_unused_layers no)
   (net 21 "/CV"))
  (pad "14" thru_hole circle (at 15.24 -2.54 270) (size 1.8034 1.8034) (drill 1.2954) (layers "*.Cu" "*.Mask") (remove_unused_layers no)
   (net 21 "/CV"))
  (pad "15" thru_hole circle (at 17.78 0 270) (size 1.8034 1.8034) (drill 1.2954) (layers "*.Cu" "*.Mask") (remove_unused_layers no)
   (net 23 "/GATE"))
  (pad "16" thru_hole circle (at 17.78 -2.54 270) (size 1.8034 1.8034) (drill 1.2954) (layers "*.Cu" "*.Mask") (remove_unused_layers no)
   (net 23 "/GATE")))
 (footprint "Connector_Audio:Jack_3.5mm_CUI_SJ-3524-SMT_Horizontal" (layer "B.Cu") (at 164.45 61.3 180)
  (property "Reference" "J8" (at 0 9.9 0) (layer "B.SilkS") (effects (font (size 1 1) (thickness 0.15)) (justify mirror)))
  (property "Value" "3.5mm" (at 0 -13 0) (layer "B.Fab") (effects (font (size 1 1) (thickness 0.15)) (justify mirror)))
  (pad "" np_thru_hole circle (at 0 -4.5 180) (size 1.7 1.7) (drill 1.7) (layers "*.Cu" "*.Mask"))
  (pad "" np_thru_hole circle (at 0 2.5 180) (size 1.7 1.7) (drill 1.7) (layers "*.Cu" "*.Mask"))
  (pad "R" smd rect (at 3.7 1.6 180) (size 2.8 2.2) (layers "B.Cu" "B.Paste" "B.Mask") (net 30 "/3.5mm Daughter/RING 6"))
  (pad "S" smd rect (at -3.7 3.6 180) (size 2.8 2.2) (layers "B.Cu" "B.Paste" "B.Mask") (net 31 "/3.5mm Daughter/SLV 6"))
  (pad "T" smd rect (at -3.7 -5.8 180) (size 2.8 2.8) (layers "B.Cu" "B.Paste" "B.Mask") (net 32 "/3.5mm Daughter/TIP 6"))
  (pad "TN" smd rect (at 0.75 -9.8 180) (size 2.8 2.6) (layers "B.Cu" "B.Paste" "B.Mask") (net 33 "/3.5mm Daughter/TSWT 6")))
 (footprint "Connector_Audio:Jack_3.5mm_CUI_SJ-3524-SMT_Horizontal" (layer "B.Cu") (at 139.95 61.3 180)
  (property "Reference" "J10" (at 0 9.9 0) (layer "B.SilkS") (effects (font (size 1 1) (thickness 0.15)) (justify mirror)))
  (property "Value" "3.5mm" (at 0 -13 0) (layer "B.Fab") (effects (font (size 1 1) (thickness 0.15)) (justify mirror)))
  (pad "" np_thru_hole circle (at 0 -4.5 180) (size 1.7 1.7) (drill 1.7) (layers "*.Cu" "*.Mask"))
  (pad "" np_thru_hole circle (at 0 2.5 180) (size 1.7 1.7) (drill 1.7) (layers "*.Cu" "*.Mask"))
  (pad "R" smd rect (at 3.7 1.6 180) (size 2.8 2.2) (layers "B.Cu" "B.Paste" "B.Mask") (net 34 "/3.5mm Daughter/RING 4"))
  (pad "S" smd rect (at -3.7 3.6 180) (size 2.8 2.2) (layers "B.Cu" "B.Paste" "B.Mask") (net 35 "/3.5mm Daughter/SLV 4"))
  (pad "T" smd rect (at -3.7 -5.8 180) (size 2.8 2.8) (layers "B.Cu" "B.Paste" "B.Mask") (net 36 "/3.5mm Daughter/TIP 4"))
  (pad "TN" smd rect (at 0.75 -9.8 180) (size 2.8 2.6) (layers "B.Cu" "B.Paste" "B.Mask") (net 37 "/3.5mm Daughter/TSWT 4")))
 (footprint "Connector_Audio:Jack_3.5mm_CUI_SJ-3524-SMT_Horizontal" (layer "B.Cu") (at 152.2 61.3 180)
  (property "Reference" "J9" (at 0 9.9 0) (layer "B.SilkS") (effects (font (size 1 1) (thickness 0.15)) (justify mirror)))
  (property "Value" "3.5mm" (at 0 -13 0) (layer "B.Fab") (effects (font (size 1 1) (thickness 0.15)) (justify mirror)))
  (pad "" np_thru_hole circle (at 0 -4.5 180) (size 1.7 1.7) (drill 1.7) (layers "*.Cu" "*.Mask"))
  (pad "" np_thru_hole circle (at 0 2.5 180) (size 1.7 1.7) (drill 1.7) (layers "*.Cu" "*.Mask"))
  (pad "R" smd rect (at 3.7 1.6 180) (size 2.8 2.2) (layers "B.Cu" "B.Paste" "B.Mask") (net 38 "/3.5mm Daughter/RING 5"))
  (pad "S" smd rect (at -3.7 3.6 180) (size 2.8 2.2) (layers "B.Cu" "B.Paste" "B.Mask") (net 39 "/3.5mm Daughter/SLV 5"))
  (pad "T" smd rect (at -3.7 -5.8 180) (size 2.8 2.8) (layers "B.Cu" "B.Paste" "B.Mask") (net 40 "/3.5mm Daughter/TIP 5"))
  (pad "TN" smd rect (at 0.75 -9.8 180) (size 2.8 2.6) (layers "B.Cu" "B.Paste" "B.Mask") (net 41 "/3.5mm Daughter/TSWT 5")))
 (gr_arc (start 206.774999 49.899793) (mid 211.017787 51.657213) (end 212.775207 55.900001) (stroke (width 0.1) (type default))
  (layer "Edge.Cuts"))
 (gr_arc (start 212.775207 134.949999) (mid 211.017787 139.192787) (end 206.774999 140.950207) (stroke (width 0.1) (type default))
  (layer "Edge.Cuts"))
 (gr_line (start 101.725 113.65) (end 42.525 113.65) (stroke (width 0.05) (type default)) (layer "Edge.Cuts"))
 (gr_line (start 212.775207 55.900001) (end 212.775207 134.949999) (stroke (width 0.1) (type default)) (layer "Edge.Cuts"))
 (gr_arc (start 113.324792 55.9) (mid 115.082212 51.657212) (end 119.325 49.899792) (stroke (width 0.1) (type default)) (layer "Edge.Cuts"))
 (gr_line (start 119.325 49.899792) (end 206.774999 49.899793) (stroke (width 0.1) (type default)) (layer "Edge.Cuts"))
 (gr_arc (start 119.325001 140.950207) (mid 115.082213 139.192787) (end 113.324793 134.949999) (stroke (width 0.1) (type default))
  (layer "Edge.Cuts"))
 (gr_line (start 205.2 140.95) (end 206.774999 140.95022) (stroke (width 0.1) (type default)) (layer "Edge.Cuts"))
 (gr_line (start 120.9 140.95) (end 119.325001 140.950207) (stroke (width 0.1) (type default)) (layer "Edge.Cuts"))
 (gr_line (start 113.324793 134.949999) (end 113.324792 55.9) (stroke (width 0.1) (type default)) (layer "Edge.Cuts"))
 (segment (start 241.179901 147.6234) (end 243.719901 147.6234) (width 0.2794) (layer "F.Cu") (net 23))
 (segment (start 241.179901 145.0834) (end 243.719901 145.0834) (width 0.2794) (layer "F.Cu") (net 21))
 (segment (start 241.179901 142.5434) (end 243.719901 142.5434) (width 2.286) (layer "F.Cu") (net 18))
 (segment (start 241.179901 140.0034) (end 243.719901 140.0034) (width 2.286) (layer "B.Cu") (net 17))
 (segment (start 241.179901 129.8434) (end 243.719901 129.8434) (width 2.286) (layer "B.Cu") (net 16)))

